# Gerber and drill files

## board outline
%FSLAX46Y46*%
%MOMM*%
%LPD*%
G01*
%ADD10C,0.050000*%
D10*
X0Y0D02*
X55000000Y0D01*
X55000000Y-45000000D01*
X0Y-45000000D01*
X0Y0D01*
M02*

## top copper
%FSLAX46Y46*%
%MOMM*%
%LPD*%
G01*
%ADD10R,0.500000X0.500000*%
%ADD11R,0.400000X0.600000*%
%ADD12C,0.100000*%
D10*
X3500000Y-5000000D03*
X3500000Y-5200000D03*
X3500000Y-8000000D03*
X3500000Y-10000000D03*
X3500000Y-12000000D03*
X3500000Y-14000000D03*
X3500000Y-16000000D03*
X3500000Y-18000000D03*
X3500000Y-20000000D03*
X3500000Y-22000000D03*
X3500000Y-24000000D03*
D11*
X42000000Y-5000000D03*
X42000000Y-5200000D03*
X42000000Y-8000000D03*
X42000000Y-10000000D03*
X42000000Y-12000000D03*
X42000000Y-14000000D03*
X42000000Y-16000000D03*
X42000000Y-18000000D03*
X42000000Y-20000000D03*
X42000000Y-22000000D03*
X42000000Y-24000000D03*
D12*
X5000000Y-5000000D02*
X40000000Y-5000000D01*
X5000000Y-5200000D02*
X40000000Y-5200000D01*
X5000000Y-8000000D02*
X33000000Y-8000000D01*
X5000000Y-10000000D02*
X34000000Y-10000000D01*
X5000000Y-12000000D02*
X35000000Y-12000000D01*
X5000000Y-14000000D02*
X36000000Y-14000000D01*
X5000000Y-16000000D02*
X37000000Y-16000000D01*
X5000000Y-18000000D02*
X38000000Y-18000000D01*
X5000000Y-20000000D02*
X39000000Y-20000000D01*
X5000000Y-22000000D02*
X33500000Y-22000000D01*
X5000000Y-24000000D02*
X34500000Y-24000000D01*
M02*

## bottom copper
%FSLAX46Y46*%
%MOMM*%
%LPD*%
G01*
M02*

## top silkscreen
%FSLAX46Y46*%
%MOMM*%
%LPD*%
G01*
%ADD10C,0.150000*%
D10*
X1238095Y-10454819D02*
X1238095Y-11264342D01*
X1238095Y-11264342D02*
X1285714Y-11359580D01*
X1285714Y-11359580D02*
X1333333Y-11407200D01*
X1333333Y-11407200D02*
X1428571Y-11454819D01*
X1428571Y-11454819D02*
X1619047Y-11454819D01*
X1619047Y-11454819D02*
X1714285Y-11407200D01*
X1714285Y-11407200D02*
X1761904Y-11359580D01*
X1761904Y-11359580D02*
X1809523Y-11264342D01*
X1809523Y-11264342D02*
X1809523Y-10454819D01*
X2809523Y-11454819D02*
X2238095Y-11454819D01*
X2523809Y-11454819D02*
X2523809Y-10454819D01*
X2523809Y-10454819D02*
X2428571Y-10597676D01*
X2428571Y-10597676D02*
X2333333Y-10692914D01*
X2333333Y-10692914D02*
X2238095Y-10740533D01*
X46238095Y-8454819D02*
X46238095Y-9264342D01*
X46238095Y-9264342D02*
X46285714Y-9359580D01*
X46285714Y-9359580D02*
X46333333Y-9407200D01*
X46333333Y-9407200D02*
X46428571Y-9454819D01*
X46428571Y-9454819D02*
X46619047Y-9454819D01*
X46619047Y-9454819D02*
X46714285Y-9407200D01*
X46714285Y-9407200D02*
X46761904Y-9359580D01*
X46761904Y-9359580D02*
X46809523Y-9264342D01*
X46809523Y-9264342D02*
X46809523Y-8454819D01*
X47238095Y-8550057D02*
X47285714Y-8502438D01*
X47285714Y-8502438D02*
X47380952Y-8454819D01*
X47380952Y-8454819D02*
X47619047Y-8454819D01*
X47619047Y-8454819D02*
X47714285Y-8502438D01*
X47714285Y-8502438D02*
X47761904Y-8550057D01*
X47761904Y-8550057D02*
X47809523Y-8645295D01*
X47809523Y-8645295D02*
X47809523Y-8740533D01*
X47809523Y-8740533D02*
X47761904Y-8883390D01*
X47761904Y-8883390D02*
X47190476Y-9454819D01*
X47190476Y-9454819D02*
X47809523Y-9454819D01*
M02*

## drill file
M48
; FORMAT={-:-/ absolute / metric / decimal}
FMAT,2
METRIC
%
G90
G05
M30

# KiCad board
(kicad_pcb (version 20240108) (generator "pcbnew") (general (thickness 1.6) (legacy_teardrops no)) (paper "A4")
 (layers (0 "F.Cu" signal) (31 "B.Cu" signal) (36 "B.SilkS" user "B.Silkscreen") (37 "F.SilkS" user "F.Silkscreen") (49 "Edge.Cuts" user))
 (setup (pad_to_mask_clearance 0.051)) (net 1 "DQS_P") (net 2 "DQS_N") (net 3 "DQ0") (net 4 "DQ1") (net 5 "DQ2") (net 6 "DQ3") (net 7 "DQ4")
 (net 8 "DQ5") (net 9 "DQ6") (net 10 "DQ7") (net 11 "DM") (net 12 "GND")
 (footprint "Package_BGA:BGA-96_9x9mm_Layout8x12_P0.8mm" (layer "F.Cu") (at 2 18)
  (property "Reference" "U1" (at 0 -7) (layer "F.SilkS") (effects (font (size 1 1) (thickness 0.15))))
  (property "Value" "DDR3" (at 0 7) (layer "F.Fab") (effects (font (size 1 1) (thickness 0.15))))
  (pad "A1" smd rect (at 1.5 -13) (size 0.5 0.5) (layers "F.Cu" "F.Paste" "F.Mask") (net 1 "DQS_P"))
  (pad "A2" smd rect (at 1.5 -12.8) (size 0.5 0.5) (layers "F.Cu" "F.Paste" "F.Mask") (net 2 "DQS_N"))
  (pad "B1" smd rect (at 1.5 -10) (size 0.5 0.5) (layers "F.Cu" "F.Paste" "F.Mask") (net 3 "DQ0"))
  (pad "B2" smd rect (at 1.5 -8) (size 0.5 0.5) (layers "F.Cu" "F.Paste" "F.Mask") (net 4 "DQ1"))
  (pad "B3" smd rect (at 1.5 -6) (size 0.5 0.5) (layers "F.Cu" "F.Paste" "F.Mask") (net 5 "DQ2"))
  (pad "B4" smd rect (at 1.5 -4) (size 0.5 0.5) (layers "F.Cu" "F.Paste" "F.Mask") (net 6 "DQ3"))
  (pad "B5" smd rect (at 1.5 -2) (size 0.5 0.5) (layers "F.Cu" "F.Paste" "F.Mask") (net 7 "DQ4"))
  (pad "B6" smd rect (at 1.5 0) (size 0.5 0.5) (layers "F.Cu" "F.Paste" "F.Mask") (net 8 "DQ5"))
  (pad "B7" smd rect (at 1.5 2) (size 0.5 0.5) (layers "F.Cu" "F.Paste" "F.Mask") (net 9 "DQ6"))
  (pad "B8" smd rect (at 1.5 4) (size 0.5 0.5) (layers "F.Cu" "F.Paste" "F.Mask") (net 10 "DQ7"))
  (pad "B9" smd rect (at 1.5 6) (size 0.5 0.5) (layers "F.Cu" "F.Paste" "F.Mask") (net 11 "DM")))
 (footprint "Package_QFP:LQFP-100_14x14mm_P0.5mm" (layer "F.Cu") (at 47 18)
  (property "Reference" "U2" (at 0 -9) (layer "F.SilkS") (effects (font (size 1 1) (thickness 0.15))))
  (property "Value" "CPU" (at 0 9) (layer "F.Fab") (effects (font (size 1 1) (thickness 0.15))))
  (pad "1" smd rect (at -5 -13) (size 0.4 0.6) (layers "F.Cu" "F.Paste" "F.Mask") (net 1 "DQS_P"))
  (pad "2" smd rect (at -5 -12.8) (size 0.4 0.6) (layers "F.Cu" "F.Paste" "F.Mask") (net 2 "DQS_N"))
  (pad "3" smd rect (at -5 -10) (size 0.4 0.6) (layers "F.Cu" "F.Paste" "F.Mask") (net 3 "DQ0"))
  (pad "4" smd rect (at -5 -8) (size 0.4 0.6) (layers "F.Cu" "F.Paste" "F.Mask") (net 4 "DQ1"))
  (pad "5" smd rect (at -5 -6) (size 0.4 0.6) (layers "F.Cu" "F.Paste" "F.Mask") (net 5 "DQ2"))
  (pad "6" smd rect (at -5 -4) (size 0.4 0.6) (layers "F.Cu" "F.Paste" "F.Mask") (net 6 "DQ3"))
  (pad "7" smd rect (at -5 -2) (size 0.4 0.6) (layers "F.Cu" "F.Paste" "F.Mask") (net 7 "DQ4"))
  (pad "8" smd rect (at -5 0) (size 0.4 0.6) (layers "F.Cu" "F.Paste" "F.Mask") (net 8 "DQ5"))
  (pad "9" smd rect (at -5 2) (size 0.4 0.6) (layers "F.Cu" "F.Paste" "F.Mask") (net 9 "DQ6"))
  (pad "10" smd rect (at -5 4) (size 0.4 0.6) (layers "F.Cu" "F.Paste" "F.Mask") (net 10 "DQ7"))
  (pad "11" smd rect (at -5 6) (size 0.4 0.6) (layers "F.Cu" "F.Paste" "F.Mask") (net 11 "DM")))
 (segment (start 5 5) (end 40 5) (width 0.1) (layer "F.Cu") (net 1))
 (segment (start 5 5.2) (end 40 5.2) (width 0.1) (layer "F.Cu") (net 2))
 (segment (start 5 8.0) (end 33.0 8.0) (width 0.1) (layer "F.Cu") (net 3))
 (segment (start 5 10.0) (end 34.0 10.0) (width 0.1) (layer "F.Cu") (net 4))
 (segment (start 5 12.0) (end 35.0 12.0) (width 0.1) (layer "F.Cu") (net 5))
 (segment (start 5 14.0) (end 36.0 14.0) (width 0.1) (layer "F.Cu") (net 6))
 (segment (start 5 16.0) (end 37.0 16.0) (width 0.1) (layer "F.Cu") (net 7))
 (segment (start 5 18.0) (end 38.0 18.0) (width 0.1) (layer "F.Cu") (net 8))
 (segment (start 5 20.0) (end 39.0 20.0) (width 0.1) (layer "F.Cu") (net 9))
 (segment (start 5 22.0) (end 33.5 22.0) (width 0.1) (layer "F.Cu") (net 10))
 (segment (start 5 24.0) (end 34.5 24.0) (width 0.1) (layer "F.Cu") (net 11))
 (gr_rect (start 0 0) (end 55 45) (layer "Edge.Cuts") (width 0.05)))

